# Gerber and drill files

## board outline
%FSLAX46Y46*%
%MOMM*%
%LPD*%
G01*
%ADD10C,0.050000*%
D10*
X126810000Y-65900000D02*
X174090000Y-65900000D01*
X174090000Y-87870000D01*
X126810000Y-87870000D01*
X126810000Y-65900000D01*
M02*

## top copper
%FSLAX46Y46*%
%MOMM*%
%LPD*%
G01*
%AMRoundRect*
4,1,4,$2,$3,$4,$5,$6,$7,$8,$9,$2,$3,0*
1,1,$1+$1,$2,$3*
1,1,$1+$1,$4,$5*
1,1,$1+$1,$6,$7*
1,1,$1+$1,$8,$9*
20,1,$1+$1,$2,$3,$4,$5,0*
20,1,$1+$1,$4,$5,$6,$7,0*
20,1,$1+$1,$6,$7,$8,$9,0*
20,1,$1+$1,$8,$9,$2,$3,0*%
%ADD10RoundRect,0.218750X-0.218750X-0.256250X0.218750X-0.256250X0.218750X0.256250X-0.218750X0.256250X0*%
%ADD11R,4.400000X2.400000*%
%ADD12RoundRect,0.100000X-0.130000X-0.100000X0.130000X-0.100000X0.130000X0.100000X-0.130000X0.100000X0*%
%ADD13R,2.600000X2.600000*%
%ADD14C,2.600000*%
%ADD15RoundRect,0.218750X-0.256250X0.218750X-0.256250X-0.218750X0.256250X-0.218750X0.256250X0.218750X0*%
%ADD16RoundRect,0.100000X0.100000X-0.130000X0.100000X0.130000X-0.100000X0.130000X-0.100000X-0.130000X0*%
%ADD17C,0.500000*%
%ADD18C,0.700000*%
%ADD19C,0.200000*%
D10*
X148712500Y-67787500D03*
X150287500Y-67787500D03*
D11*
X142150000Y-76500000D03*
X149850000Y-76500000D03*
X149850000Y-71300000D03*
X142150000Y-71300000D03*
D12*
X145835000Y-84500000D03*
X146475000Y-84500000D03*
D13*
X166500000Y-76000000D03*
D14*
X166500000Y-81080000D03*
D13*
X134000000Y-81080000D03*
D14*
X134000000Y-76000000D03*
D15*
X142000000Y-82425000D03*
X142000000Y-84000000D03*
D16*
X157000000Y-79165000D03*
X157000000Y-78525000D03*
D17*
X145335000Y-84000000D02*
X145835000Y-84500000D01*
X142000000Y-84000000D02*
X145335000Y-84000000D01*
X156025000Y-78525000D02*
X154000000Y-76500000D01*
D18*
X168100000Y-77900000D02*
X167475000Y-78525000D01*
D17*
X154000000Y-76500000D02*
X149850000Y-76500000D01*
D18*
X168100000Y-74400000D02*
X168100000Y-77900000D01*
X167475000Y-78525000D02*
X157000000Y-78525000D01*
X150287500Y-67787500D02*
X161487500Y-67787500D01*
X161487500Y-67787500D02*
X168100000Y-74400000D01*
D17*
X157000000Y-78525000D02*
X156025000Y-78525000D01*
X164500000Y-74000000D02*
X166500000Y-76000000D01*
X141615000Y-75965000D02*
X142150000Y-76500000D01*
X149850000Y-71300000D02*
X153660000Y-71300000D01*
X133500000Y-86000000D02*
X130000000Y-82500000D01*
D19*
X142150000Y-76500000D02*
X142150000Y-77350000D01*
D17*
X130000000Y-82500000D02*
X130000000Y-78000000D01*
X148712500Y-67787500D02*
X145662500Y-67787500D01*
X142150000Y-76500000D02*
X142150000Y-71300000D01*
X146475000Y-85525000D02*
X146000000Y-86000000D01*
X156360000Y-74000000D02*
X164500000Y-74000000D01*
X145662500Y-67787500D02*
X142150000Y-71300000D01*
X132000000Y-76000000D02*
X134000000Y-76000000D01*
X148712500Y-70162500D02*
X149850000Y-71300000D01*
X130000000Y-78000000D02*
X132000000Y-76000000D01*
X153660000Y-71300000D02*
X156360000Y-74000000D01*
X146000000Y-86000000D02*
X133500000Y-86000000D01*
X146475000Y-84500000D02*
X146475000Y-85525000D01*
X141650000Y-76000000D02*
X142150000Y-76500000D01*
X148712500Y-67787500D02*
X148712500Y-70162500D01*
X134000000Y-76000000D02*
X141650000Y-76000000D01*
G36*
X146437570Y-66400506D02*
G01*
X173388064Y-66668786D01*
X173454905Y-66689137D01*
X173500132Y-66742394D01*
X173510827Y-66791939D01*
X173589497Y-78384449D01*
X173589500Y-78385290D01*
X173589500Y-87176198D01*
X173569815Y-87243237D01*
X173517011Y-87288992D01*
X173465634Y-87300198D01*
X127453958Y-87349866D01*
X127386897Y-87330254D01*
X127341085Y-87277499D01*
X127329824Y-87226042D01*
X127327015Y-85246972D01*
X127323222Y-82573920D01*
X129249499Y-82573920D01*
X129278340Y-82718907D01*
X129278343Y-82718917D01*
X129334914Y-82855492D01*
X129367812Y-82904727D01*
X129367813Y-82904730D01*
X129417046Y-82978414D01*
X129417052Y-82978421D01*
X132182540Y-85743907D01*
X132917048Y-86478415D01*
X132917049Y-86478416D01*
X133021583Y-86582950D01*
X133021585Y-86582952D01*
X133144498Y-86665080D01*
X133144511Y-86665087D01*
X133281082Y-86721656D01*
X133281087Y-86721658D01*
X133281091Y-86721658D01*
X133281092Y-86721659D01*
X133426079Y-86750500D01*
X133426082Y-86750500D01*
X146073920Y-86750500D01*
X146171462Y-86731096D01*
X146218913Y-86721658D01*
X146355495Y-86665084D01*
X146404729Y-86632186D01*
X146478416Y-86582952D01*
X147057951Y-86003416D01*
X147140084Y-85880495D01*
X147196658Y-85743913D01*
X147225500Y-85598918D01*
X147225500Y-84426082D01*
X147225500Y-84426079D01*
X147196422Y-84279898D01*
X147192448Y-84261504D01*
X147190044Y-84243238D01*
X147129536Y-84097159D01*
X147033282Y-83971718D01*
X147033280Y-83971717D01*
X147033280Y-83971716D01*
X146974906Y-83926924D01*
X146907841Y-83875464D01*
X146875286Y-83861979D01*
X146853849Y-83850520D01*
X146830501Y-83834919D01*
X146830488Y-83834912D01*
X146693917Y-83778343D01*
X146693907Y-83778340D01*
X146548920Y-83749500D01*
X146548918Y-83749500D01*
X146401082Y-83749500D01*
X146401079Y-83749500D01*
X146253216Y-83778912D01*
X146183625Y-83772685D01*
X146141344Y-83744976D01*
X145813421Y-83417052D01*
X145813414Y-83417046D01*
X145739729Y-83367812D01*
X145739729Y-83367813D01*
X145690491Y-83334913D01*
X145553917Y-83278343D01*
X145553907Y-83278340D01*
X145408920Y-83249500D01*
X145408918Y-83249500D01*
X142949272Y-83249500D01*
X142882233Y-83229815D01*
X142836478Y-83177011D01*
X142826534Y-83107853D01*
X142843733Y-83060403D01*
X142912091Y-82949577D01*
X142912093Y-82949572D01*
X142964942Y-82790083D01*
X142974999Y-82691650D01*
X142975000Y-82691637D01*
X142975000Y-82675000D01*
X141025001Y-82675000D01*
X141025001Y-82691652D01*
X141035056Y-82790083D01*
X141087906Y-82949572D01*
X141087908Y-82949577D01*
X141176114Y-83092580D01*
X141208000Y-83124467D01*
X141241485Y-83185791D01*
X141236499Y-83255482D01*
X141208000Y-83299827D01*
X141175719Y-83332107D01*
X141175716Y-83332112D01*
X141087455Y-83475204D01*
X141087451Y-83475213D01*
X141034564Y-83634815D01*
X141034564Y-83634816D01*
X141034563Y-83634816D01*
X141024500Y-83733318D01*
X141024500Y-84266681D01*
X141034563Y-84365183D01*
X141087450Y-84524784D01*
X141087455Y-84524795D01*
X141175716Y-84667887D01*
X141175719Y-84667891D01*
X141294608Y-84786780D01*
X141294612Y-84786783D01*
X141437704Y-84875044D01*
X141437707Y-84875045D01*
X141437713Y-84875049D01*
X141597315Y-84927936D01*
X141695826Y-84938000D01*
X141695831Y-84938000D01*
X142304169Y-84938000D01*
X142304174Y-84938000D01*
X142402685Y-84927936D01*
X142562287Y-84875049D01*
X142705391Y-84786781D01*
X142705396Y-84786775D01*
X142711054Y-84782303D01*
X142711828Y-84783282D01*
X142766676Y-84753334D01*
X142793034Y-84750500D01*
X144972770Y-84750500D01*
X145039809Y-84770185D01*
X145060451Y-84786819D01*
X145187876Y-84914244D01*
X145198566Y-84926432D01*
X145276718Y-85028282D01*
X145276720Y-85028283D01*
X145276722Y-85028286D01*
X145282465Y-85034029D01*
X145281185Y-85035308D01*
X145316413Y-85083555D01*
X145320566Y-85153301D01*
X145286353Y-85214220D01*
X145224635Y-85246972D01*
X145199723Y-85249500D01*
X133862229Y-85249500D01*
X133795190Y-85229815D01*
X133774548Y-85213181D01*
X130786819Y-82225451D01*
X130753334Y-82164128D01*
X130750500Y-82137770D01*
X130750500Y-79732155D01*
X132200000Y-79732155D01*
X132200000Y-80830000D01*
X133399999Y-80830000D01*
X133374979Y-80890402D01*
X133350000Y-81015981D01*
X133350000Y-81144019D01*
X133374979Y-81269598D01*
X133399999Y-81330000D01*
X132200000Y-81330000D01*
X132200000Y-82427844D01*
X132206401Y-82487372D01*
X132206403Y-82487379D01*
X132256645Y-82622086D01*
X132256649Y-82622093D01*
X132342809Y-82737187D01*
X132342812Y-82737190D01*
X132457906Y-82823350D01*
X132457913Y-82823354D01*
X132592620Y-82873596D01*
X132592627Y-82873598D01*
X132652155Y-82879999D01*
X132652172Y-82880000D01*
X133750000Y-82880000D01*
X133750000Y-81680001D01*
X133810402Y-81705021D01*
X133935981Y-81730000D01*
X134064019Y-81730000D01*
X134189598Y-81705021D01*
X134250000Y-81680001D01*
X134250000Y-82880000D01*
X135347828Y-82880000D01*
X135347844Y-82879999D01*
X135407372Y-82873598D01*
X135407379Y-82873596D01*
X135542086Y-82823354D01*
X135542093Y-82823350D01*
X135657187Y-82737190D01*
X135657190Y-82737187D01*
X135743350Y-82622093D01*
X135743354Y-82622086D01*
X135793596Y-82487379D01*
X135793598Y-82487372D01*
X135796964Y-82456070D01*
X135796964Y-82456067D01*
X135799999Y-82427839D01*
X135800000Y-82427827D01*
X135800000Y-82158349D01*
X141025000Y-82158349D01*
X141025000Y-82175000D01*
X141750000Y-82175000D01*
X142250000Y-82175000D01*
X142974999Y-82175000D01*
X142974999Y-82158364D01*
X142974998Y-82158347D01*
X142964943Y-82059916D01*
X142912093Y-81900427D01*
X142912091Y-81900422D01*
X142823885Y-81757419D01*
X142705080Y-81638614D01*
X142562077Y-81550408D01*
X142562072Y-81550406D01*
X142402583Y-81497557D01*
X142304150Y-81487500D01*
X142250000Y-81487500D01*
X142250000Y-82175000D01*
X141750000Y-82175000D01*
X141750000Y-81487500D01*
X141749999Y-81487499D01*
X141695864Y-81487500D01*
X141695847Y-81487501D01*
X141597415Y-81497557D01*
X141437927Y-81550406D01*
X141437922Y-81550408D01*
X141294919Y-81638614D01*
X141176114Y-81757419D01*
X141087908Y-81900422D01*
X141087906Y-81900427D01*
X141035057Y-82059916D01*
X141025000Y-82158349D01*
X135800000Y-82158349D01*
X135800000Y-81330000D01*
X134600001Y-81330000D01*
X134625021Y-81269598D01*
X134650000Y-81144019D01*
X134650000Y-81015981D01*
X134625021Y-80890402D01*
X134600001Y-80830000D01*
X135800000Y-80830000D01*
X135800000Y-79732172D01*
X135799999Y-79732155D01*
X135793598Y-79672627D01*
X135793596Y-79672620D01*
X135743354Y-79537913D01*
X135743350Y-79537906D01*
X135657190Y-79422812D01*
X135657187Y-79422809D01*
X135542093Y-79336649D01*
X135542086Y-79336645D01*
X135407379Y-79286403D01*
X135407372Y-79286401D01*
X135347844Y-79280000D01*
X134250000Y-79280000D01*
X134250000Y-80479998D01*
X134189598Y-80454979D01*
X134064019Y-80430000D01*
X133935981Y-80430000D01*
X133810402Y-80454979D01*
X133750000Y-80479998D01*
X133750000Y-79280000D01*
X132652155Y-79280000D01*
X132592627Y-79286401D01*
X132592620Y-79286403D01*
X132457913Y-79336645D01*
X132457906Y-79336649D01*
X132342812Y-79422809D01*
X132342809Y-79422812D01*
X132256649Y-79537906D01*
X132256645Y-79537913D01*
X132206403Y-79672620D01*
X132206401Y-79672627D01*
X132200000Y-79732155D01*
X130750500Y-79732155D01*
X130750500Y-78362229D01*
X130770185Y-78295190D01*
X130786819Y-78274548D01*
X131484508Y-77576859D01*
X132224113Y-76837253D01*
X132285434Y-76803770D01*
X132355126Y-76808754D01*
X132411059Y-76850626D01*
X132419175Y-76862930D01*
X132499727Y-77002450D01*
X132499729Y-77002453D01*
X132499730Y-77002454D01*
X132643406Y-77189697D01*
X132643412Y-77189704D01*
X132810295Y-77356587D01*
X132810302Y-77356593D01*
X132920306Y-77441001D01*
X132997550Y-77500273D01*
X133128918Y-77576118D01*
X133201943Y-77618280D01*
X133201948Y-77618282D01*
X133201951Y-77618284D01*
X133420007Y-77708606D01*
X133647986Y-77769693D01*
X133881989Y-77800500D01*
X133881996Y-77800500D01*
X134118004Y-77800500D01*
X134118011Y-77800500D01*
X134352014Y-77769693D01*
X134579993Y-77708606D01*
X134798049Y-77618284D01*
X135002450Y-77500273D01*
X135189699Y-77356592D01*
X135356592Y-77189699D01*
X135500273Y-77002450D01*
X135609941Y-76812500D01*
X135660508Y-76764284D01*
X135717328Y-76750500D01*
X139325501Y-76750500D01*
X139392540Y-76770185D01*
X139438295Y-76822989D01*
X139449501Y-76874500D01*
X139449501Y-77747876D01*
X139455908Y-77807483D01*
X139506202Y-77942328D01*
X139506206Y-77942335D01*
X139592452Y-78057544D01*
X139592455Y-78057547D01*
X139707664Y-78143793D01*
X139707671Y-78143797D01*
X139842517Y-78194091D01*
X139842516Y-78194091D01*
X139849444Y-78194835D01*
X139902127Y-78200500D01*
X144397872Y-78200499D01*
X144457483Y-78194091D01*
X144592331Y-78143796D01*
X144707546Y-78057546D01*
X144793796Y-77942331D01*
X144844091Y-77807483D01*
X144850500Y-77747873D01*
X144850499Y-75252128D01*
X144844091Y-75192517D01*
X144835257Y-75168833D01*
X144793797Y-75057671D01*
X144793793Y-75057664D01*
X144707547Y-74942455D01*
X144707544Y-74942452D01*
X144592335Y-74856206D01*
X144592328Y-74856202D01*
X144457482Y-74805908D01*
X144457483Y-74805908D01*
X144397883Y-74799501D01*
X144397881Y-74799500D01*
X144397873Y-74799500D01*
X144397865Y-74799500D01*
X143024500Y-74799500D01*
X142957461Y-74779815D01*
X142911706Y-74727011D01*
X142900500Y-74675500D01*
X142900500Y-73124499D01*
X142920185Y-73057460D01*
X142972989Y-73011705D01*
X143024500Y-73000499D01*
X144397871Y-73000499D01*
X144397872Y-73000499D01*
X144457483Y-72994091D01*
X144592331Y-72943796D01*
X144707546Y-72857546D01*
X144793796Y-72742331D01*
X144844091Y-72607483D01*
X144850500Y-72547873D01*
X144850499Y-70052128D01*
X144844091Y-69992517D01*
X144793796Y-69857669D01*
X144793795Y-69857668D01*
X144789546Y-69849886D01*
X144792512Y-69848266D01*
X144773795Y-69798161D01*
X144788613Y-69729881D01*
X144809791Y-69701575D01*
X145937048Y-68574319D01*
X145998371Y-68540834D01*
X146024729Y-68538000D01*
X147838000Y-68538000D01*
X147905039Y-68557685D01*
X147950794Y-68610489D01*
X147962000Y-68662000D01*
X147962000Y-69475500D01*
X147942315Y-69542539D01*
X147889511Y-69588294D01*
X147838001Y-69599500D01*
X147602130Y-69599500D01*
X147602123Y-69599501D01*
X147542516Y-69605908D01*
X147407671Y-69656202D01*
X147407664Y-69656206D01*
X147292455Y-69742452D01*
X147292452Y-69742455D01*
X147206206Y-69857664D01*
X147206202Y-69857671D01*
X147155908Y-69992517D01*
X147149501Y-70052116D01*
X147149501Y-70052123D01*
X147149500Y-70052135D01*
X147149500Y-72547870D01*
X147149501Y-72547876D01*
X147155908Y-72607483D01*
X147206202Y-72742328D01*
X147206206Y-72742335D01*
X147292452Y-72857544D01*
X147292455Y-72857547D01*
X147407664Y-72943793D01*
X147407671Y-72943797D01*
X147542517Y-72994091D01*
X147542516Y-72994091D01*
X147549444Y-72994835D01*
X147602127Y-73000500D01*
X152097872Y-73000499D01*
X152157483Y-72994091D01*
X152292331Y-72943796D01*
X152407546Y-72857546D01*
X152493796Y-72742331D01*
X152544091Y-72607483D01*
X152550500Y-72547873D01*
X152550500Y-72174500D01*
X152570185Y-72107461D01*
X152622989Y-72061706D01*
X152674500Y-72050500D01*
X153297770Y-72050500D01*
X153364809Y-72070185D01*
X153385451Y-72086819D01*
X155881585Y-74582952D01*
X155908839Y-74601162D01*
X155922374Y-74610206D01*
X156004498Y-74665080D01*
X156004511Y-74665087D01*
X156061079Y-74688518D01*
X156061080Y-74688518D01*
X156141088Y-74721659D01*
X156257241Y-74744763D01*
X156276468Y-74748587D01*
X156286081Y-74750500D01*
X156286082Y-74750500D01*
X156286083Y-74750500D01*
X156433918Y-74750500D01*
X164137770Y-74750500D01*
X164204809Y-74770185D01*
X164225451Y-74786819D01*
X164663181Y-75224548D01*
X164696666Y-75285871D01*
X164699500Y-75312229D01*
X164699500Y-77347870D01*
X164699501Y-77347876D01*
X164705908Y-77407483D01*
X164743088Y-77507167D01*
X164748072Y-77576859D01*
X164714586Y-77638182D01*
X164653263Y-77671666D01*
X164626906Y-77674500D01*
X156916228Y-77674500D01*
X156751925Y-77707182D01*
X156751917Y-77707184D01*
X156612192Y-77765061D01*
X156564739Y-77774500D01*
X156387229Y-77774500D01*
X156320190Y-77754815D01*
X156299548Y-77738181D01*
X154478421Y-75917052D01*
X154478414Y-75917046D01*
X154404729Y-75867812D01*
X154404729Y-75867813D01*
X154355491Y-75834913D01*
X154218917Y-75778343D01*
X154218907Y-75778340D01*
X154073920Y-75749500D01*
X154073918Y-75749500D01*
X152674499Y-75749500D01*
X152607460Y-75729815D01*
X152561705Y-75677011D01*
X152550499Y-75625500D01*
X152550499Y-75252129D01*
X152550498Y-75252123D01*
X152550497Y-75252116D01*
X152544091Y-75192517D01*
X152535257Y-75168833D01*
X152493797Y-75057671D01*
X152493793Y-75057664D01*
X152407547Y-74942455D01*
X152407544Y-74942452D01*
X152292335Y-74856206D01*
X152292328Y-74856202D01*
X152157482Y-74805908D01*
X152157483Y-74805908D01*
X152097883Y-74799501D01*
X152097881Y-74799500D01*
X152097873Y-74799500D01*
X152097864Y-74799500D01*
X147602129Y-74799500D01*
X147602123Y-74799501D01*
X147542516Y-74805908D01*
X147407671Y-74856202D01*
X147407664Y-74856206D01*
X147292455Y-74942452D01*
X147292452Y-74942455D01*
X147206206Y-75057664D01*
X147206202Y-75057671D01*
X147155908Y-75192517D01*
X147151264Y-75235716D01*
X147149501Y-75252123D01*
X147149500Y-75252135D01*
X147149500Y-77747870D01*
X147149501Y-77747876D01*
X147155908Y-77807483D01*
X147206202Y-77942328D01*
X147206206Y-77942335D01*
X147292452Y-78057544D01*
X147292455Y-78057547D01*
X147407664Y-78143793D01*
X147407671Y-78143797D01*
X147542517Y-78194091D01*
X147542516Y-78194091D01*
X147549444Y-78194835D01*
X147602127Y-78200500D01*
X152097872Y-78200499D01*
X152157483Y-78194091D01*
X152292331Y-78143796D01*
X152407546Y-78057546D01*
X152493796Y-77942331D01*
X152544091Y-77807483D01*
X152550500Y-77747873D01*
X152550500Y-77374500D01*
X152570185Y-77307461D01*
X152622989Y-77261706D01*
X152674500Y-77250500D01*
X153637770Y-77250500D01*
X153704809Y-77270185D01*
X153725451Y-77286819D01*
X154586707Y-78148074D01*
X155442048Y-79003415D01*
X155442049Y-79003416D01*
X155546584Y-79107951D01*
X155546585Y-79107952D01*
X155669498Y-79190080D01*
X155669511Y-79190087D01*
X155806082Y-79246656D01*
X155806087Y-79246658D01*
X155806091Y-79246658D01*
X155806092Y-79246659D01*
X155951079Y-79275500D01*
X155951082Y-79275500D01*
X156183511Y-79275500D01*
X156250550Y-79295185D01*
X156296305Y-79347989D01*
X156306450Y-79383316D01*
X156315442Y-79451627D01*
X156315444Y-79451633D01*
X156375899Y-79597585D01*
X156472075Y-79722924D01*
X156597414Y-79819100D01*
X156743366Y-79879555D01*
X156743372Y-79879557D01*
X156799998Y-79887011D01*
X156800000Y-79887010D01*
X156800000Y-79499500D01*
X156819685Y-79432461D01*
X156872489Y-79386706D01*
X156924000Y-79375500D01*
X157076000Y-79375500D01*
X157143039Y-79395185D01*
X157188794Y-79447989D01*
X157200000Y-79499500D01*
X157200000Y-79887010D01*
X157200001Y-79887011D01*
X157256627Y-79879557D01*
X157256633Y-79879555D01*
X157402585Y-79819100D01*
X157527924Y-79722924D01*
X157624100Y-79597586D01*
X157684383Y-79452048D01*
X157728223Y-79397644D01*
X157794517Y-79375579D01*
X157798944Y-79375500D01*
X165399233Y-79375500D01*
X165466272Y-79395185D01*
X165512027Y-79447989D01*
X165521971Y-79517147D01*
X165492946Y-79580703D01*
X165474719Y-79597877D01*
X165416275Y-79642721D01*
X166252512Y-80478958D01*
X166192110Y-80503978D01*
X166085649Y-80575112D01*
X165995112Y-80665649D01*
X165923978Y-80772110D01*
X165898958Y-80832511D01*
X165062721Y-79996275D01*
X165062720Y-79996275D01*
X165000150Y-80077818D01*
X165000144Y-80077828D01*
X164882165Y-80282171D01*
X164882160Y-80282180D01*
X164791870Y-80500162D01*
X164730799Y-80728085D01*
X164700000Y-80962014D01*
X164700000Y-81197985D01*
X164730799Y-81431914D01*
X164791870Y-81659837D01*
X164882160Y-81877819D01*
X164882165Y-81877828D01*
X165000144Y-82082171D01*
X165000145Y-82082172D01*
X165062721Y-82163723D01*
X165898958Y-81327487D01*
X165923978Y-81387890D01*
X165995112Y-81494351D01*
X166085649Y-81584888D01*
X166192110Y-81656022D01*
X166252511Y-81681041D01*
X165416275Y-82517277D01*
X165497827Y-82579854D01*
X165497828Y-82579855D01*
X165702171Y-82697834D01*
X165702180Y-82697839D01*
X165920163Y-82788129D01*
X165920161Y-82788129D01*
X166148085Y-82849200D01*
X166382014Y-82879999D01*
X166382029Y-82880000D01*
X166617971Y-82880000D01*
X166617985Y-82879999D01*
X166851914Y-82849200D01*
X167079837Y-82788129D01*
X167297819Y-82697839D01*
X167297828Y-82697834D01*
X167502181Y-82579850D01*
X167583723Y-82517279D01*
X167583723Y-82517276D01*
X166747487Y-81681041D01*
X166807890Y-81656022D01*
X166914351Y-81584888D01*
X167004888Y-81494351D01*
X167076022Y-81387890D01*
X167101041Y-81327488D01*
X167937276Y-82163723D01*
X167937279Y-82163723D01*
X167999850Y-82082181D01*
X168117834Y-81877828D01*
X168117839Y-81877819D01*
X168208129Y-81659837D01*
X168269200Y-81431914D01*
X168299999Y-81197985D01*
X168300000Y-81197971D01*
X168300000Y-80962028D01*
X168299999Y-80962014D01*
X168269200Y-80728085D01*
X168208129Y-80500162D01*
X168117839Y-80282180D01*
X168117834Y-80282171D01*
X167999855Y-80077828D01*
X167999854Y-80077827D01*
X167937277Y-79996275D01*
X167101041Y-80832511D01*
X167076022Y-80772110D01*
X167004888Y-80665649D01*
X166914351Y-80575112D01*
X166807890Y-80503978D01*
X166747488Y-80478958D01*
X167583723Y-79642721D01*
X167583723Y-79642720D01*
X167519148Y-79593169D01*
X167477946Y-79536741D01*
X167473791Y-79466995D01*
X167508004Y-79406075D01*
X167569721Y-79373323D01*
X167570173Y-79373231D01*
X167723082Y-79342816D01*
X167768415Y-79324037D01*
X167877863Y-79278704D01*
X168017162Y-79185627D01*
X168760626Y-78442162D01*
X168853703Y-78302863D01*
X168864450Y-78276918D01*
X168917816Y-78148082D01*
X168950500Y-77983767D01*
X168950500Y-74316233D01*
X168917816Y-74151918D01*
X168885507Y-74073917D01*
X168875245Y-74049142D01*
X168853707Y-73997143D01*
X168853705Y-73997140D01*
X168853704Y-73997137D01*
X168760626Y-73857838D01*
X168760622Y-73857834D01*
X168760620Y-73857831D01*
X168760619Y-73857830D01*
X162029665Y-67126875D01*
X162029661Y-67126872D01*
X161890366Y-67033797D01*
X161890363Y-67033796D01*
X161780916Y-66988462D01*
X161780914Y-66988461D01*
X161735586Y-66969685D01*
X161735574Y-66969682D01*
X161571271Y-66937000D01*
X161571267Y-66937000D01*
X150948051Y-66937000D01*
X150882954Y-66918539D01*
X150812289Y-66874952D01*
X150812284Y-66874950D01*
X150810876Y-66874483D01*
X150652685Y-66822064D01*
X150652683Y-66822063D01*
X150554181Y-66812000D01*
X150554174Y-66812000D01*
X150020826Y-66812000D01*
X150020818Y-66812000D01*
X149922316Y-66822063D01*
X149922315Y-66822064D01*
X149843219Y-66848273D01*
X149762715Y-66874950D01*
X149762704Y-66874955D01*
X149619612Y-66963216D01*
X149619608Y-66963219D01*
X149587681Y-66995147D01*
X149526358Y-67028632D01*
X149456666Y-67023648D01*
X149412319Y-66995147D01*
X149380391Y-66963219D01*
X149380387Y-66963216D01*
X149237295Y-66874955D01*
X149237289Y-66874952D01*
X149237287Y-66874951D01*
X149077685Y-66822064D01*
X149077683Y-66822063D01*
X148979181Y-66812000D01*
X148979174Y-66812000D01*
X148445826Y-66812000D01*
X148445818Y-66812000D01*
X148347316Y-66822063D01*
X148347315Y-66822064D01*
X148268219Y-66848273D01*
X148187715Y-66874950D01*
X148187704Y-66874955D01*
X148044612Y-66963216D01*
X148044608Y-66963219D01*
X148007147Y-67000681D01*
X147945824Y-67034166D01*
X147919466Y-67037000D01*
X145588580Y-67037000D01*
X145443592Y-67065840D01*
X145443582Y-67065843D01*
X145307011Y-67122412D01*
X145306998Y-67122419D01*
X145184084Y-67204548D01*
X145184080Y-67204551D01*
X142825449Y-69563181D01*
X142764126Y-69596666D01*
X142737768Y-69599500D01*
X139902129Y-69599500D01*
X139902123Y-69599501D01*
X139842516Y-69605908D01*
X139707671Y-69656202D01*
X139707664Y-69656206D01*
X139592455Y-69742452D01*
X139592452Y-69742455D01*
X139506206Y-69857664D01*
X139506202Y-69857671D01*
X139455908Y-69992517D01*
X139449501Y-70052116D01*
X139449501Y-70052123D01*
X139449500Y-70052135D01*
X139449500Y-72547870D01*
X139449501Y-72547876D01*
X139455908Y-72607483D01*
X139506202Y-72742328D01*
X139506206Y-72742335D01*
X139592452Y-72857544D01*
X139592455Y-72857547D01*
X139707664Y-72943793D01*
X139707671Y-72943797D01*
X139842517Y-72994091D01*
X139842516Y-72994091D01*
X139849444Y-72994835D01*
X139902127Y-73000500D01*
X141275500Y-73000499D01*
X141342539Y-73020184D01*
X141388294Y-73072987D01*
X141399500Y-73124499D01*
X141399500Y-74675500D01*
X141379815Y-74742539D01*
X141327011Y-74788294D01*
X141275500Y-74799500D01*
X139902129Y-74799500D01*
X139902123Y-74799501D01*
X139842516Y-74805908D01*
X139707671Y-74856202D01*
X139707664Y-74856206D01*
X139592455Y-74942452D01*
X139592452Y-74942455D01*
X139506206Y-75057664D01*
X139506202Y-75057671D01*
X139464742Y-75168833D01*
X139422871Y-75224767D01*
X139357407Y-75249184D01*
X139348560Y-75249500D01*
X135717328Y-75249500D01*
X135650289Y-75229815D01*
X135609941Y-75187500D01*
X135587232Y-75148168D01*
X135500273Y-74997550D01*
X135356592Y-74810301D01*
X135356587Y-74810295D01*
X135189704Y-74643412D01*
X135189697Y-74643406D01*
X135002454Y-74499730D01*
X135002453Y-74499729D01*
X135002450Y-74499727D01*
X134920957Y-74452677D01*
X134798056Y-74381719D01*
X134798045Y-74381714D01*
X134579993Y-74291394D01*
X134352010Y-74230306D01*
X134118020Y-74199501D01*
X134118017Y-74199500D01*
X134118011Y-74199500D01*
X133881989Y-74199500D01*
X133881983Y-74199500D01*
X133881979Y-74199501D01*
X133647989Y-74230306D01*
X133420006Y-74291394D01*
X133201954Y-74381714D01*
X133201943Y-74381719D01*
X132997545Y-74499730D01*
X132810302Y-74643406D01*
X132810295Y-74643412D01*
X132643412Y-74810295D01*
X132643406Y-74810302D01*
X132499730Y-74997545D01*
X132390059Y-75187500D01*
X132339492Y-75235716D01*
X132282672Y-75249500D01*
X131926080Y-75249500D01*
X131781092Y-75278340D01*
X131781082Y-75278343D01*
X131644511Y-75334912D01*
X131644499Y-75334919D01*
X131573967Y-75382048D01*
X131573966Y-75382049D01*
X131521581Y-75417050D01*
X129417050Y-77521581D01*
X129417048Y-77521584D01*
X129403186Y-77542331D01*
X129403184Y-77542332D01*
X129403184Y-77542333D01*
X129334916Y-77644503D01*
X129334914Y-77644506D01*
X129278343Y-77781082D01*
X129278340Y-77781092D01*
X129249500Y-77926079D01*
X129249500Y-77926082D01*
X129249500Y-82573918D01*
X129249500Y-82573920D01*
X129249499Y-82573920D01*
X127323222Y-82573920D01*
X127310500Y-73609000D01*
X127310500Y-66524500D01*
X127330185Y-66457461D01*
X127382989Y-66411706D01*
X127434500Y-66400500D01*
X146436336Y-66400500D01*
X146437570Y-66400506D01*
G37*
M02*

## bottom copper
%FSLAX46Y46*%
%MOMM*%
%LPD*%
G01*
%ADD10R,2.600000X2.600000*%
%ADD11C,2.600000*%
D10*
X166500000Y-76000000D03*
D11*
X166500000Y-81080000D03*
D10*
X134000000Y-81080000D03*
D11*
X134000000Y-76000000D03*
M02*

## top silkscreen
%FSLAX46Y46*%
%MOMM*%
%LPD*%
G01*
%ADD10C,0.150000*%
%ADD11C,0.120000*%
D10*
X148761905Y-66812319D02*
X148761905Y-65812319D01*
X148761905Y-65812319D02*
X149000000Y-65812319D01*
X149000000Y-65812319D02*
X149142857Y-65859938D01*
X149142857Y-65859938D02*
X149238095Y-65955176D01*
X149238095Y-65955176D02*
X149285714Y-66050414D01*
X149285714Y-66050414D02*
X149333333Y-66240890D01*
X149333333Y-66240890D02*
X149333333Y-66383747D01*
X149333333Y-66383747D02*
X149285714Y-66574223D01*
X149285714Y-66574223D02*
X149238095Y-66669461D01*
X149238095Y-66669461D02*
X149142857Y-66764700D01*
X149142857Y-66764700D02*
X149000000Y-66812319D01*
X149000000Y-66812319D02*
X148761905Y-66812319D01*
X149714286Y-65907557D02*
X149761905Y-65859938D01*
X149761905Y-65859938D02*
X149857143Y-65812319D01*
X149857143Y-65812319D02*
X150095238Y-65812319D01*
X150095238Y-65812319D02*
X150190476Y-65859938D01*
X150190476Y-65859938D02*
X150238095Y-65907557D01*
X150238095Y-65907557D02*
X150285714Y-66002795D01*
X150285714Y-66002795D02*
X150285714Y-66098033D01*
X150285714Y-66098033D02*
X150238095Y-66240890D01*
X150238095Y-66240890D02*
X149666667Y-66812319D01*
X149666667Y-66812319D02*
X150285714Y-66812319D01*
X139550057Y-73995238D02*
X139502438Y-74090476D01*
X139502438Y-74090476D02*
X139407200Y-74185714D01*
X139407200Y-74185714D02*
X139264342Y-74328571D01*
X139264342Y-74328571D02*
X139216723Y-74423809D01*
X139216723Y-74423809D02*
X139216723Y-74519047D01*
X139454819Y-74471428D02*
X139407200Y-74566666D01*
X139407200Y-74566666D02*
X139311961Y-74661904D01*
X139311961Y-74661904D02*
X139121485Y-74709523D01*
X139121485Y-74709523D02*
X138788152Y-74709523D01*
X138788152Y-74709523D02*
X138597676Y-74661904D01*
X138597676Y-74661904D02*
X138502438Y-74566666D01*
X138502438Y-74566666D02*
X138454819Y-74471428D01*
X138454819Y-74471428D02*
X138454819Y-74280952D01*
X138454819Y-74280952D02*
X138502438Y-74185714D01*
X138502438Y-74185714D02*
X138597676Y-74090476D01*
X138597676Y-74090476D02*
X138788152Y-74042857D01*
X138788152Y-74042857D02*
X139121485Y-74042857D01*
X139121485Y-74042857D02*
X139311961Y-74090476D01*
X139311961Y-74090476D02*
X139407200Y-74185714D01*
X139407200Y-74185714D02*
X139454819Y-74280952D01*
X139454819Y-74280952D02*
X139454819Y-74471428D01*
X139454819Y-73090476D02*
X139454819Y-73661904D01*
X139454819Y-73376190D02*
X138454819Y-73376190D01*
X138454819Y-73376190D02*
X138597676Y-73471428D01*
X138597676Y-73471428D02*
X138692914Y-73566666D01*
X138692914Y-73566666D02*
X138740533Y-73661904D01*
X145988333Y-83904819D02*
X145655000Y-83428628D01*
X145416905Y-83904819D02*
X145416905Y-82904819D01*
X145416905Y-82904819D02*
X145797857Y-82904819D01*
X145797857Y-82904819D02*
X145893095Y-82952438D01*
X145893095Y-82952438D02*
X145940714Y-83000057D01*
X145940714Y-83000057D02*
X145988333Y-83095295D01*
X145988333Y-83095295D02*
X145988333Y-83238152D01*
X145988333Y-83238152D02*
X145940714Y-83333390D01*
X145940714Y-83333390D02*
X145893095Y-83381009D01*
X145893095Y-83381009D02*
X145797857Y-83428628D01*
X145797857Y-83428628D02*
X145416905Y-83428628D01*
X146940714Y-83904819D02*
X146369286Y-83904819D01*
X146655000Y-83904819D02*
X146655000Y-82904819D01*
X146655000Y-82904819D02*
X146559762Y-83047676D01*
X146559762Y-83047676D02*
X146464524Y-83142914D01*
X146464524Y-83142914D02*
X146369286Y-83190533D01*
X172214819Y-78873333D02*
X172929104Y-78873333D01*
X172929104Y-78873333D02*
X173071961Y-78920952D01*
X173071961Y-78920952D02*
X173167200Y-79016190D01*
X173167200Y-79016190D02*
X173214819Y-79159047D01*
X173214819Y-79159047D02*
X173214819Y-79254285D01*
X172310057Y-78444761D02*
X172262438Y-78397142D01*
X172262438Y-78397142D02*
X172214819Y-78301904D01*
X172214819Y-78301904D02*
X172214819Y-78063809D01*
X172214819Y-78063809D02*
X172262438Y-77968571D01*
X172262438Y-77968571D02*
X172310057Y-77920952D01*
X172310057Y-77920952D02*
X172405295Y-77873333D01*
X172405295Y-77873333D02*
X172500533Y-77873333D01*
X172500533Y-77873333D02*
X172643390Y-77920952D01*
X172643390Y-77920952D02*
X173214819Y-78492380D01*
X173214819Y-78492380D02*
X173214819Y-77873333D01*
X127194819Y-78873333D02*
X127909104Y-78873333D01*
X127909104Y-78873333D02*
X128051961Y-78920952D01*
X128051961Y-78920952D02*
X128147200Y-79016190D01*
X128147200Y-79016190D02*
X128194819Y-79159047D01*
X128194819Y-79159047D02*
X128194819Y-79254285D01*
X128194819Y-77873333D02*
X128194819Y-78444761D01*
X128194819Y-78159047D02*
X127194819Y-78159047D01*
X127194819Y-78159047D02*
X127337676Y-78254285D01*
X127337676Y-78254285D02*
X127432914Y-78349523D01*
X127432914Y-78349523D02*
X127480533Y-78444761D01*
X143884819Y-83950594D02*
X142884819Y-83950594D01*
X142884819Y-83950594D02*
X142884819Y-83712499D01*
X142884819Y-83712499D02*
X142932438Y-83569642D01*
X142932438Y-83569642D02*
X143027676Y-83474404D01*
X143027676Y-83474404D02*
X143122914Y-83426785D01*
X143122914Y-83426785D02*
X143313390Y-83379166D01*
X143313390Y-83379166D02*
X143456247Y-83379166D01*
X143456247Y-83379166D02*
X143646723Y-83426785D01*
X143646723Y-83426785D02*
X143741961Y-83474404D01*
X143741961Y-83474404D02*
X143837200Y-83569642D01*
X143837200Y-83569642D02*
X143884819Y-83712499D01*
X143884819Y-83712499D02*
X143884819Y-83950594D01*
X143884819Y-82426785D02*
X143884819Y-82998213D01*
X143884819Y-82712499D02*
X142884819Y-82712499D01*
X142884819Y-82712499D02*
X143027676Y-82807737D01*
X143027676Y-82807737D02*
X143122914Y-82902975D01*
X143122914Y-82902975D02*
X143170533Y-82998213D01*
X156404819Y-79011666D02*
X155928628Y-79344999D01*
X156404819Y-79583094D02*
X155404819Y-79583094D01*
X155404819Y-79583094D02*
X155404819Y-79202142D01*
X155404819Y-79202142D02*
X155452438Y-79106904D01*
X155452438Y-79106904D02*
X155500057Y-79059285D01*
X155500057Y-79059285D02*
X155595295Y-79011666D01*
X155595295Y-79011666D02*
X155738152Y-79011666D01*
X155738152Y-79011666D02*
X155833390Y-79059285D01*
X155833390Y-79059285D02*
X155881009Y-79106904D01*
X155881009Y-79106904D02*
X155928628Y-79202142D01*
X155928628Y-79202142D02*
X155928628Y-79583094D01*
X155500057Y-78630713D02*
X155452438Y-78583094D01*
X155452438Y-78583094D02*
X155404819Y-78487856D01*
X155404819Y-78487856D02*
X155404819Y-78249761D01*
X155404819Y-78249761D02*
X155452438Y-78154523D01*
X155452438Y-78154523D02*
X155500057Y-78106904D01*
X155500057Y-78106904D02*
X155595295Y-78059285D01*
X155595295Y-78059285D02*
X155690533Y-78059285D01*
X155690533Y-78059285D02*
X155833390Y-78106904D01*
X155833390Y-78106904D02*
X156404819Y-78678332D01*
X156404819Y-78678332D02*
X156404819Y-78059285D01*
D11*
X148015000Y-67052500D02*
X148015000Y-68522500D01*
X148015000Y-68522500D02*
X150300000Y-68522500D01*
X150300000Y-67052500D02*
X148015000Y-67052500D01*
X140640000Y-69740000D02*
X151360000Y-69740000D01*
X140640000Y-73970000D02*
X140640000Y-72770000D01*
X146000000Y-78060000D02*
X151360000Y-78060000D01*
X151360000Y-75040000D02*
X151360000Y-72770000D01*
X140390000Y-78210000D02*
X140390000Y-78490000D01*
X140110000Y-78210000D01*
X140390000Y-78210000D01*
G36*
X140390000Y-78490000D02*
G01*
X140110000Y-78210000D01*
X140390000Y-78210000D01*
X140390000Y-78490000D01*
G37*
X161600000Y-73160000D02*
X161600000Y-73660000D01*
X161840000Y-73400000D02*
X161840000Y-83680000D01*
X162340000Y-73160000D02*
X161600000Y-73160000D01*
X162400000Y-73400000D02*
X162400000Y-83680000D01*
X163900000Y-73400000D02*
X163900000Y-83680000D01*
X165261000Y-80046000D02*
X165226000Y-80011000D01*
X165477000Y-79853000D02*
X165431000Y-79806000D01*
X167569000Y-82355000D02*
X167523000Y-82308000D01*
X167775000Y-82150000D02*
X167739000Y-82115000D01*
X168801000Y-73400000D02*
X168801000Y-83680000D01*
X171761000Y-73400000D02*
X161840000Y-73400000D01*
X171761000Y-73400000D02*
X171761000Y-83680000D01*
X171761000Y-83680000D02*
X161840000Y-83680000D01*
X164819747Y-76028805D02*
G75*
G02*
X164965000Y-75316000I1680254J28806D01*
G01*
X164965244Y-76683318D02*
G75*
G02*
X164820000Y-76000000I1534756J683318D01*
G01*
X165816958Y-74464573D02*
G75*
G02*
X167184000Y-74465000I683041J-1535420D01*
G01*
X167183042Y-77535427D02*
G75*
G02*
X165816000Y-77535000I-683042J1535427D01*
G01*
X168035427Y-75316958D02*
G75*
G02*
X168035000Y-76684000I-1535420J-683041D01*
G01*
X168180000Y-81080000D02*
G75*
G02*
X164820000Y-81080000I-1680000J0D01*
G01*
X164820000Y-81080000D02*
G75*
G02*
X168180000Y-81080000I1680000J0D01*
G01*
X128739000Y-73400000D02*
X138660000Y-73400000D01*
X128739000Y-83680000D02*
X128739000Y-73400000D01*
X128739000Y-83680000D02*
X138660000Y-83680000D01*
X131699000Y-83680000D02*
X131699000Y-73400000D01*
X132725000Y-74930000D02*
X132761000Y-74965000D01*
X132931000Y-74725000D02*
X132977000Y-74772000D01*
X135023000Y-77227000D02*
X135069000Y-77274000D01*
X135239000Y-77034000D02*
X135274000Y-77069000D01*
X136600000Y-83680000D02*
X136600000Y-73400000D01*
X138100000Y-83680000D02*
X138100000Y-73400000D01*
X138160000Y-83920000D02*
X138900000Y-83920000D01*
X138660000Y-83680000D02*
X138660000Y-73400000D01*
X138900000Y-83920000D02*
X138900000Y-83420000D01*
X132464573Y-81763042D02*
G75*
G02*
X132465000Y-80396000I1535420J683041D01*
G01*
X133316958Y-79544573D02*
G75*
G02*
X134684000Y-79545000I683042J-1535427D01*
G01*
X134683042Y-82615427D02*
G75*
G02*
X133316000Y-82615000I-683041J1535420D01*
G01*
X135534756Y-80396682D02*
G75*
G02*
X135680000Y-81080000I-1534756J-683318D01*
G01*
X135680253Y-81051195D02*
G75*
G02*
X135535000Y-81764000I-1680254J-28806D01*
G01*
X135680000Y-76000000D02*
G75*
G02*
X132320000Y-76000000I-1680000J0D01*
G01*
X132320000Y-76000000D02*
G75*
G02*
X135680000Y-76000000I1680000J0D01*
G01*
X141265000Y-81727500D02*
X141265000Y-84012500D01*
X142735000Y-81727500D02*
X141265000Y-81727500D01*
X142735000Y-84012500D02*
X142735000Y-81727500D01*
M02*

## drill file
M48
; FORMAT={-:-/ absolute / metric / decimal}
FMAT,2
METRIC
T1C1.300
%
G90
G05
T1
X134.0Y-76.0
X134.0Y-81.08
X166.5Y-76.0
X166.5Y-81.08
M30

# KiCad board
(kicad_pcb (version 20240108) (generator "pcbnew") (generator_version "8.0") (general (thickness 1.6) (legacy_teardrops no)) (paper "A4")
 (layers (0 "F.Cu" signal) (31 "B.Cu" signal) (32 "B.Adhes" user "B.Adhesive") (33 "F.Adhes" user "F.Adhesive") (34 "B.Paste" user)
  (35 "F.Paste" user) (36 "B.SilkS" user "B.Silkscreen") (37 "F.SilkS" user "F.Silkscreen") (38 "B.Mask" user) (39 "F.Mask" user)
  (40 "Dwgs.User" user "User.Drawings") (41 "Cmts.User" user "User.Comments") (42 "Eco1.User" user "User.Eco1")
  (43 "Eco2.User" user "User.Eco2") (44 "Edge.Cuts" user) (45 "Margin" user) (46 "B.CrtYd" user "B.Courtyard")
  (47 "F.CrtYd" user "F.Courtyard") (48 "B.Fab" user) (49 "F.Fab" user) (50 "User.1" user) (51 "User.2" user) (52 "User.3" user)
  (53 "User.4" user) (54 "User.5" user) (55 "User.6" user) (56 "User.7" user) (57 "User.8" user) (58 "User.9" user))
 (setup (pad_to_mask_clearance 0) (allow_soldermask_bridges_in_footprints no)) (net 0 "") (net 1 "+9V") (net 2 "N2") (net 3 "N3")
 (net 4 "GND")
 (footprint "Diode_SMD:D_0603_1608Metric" (layer "F.Cu") (at 149.5 67.7875)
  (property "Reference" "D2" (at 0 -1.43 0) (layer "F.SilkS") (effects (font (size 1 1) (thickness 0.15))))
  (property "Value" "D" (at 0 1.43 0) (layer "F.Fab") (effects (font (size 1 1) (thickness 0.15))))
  (fp_line (start -1.485 -0.735) (end -1.485 0.735) (stroke (width 0.12) (type solid)) (layer "F.SilkS"))
  (fp_line (start -1.485 0.735) (end 0.8 0.735) (stroke (width 0.12) (type solid)) (layer "F.SilkS"))
  (fp_line (start 0.8 -0.735) (end -1.485 -0.735) (stroke (width 0.12) (type solid)) (layer "F.SilkS"))
  (pad "1" smd roundrect (at -0.7875 0) (size 0.875 0.95) (layers "F.Cu" "F.Paste" "F.Mask") (roundrect_rratio 0.25) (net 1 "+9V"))
  (pad "2" smd roundrect (at 0.7875 0) (size 0.875 0.95) (layers "F.Cu" "F.Paste" "F.Mask") (roundrect_rratio 0.25) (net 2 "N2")))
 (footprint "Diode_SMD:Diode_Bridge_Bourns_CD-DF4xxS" (layer "F.Cu") (at 146 73.9 90)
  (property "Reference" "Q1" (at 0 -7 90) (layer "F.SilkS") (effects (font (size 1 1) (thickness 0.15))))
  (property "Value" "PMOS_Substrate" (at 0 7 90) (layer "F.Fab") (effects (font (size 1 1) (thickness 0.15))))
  (fp_line (start 4.16 -5.36) (end 4.16 5.36) (stroke (width 0.12) (type solid)) (layer "F.SilkS"))
  (fp_line (start -0.07 -5.36) (end 1.13 -5.36) (stroke (width 0.12) (type solid)) (layer "F.SilkS"))
  (fp_line (start -4.16 0) (end -4.16 5.36) (stroke (width 0.12) (type solid)) (layer "F.SilkS"))
  (fp_line (start -1.14 5.36) (end 1.13 5.36) (stroke (width 0.12) (type solid)) (layer "F.SilkS"))
  (fp_poly
   (pts (xy -4.31 -5.61) (xy -4.59 -5.61) (xy -4.31 -5.89) (xy -4.31 -5.61)) (stroke (width 0.12) (type solid)) (fill solid)
   (layer "F.SilkS"))
  (pad "1" smd rect (at -2.6 -3.85 90) (size 2.4 4.4) (layers "F.Cu" "F.Paste" "F.Mask") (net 1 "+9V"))
  (pad "2" smd rect (at -2.6 3.85 90) (size 2.4 4.4) (layers "F.Cu" "F.Paste" "F.Mask") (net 2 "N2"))
  (pad "3" smd rect (at 2.6 3.85 90) (size 2.4 4.4) (layers "F.Cu" "F.Paste" "F.Mask") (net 1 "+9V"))
  (pad "4" smd rect (at 2.6 -3.85 90) (size 2.4 4.4) (layers "F.Cu" "F.Paste" "F.Mask") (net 1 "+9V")))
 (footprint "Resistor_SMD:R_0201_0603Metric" (layer "F.Cu") (at 146.155 84.5)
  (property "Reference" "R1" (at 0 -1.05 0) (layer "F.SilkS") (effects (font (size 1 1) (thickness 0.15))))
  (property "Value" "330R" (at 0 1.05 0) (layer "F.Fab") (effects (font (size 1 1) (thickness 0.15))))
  (pad "" smd roundrect (at -0.345 0) (size 0.318 0.36) (layers "F.Paste") (roundrect_rratio 0.25))
  (pad "" smd roundrect (at 0.345 0) (size 0.318 0.36) (layers "F.Paste") (roundrect_rratio 0.25))
  (pad "1" smd roundrect (at -0.32 0) (size 0.46 0.4) (layers "F.Cu" "F.Mask") (roundrect_rratio 0.25) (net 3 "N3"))
  (pad "2" smd roundrect (at 0.32 0) (size 0.46 0.4) (layers "F.Cu" "F.Mask") (roundrect_rratio 0.25) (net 1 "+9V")))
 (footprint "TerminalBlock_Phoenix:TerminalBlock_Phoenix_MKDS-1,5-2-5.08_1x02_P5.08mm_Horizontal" (layer "F.Cu") (at 166.5 76 -90)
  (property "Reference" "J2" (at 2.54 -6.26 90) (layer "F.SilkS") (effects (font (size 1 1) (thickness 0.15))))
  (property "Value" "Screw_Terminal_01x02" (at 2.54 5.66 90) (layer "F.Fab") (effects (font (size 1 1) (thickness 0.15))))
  (fp_line (start -2.84 4.9) (end -2.34 4.9) (stroke (width 0.12) (type solid)) (layer "F.SilkS"))
  (fp_line (start -2.6 4.66) (end 7.68 4.66) (stroke (width 0.12) (type solid)) (layer "F.SilkS"))
  (fp_line (start -2.84 4.16) (end -2.84 4.9) (stroke (width 0.12) (type solid)) (layer "F.SilkS"))
  (fp_line (start -2.6 4.1) (end 7.68 4.1) (stroke (width 0.12) (type solid)) (layer "F.SilkS"))
  (fp_line (start -2.6 2.6) (end 7.68 2.6) (stroke (width 0.12) (type solid)) (layer "F.SilkS"))
  (fp_line (start 4.046 1.239) (end 4.011 1.274) (stroke (width 0.12) (type solid)) (layer "F.SilkS"))
  (fp_line (start 3.853 1.023) (end 3.806 1.069) (stroke (width 0.12) (type solid)) (layer "F.SilkS"))
  (fp_line (start 6.355 -1.069) (end 6.308 -1.023) (stroke (width 0.12) (type solid)) (layer "F.SilkS"))
  (fp_line (start 6.15 -1.275) (end 6.115 -1.239) (stroke (width 0.12) (type solid)) (layer "F.SilkS"))
  (fp_line (start -2.6 -2.301) (end 7.68 -2.301) (stroke (width 0.12) (type solid)) (layer "F.SilkS"))
  (fp_line (start -2.6 -5.261) (end -2.6 4.66) (stroke (width 0.12) (type solid)) (layer "F.SilkS"))
  (fp_line (start -2.6 -5.261) (end 7.68 -5.261) (stroke (width 0.12) (type solid)) (layer "F.SilkS"))
  (fp_line (start 7.68 -5.261) (end 7.68 4.66) (stroke (width 0.12) (type solid)) (layer "F.SilkS"))
  (fp_arc (start 0.028805 1.680253) (mid -0.335551 1.646659) (end -0.684 1.535) (stroke (width 0.12) (type solid)) (layer "F.SilkS"))
  (fp_arc (start 0.683318 1.534756) (mid 0.349292 1.643288) (end 0 1.68) (stroke (width 0.12) (type solid)) (layer "F.SilkS"))
  (fp_arc (start -1.535427 0.683042) (mid -1.680501 -0.000524) (end -1.535 -0.684) (stroke (width 0.12) (type solid)) (layer "F.SilkS"))
  (fp_arc (start 1.535427 -0.683042) (mid 1.680501 0.000524) (end 1.535 0.684) (stroke (width 0.12) (type solid)) (layer "F.SilkS"))
  (fp_arc (start -0.683042 -1.535427) (mid 0.000524 -1.680501) (end 0.684 -1.535) (stroke (width 0.12) (type solid)) (layer "F.SilkS"))
  (fp_circle (center 5.08 0) (end 6.76 0) (stroke (width 0.12) (type solid)) (fill none) (layer "F.SilkS"))
  (pad "1" thru_hole rect (at 0 0 270) (size 2.6 2.6) (drill 1.3) (layers "*.Cu" "*.Mask") (remove_unused_layers no) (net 1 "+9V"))
  (pad "2" thru_hole circle (at 5.08 0 270) (size 2.6 2.6) (drill 1.3) (layers "*.Cu" "*.Mask") (remove_unused_layers no) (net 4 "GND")))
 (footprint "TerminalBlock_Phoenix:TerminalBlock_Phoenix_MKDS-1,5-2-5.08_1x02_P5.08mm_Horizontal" (layer "F.Cu") (at 134 81.08 90)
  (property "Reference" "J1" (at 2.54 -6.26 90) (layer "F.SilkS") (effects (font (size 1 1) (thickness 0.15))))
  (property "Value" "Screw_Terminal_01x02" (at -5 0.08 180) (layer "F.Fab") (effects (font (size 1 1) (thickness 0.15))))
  (fp_line (start 7.68 -5.261) (end 7.68 4.66) (stroke (width 0.12) (type solid)) (layer "F.SilkS"))
  (fp_line (start -2.6 -5.261) (end 7.68 -5.261) (stroke (width 0.12) (type solid)) (layer "F.SilkS"))
  (fp_line (start -2.6 -5.261) (end -2.6 4.66) (stroke (width 0.12) (type solid)) (layer "F.SilkS"))
  (fp_line (start -2.6 -2.301) (end 7.68 -2.301) (stroke (width 0.12) (type solid)) (layer "F.SilkS"))
  (fp_line (start 6.15 -1.275) (end 6.115 -1.239) (stroke (width 0.12) (type solid)) (layer "F.SilkS"))
  (fp_line (start 6.355 -1.069) (end 6.308 -1.023) (stroke (width 0.12) (type solid)) (layer "F.SilkS"))
  (fp_line (start 3.853 1.023) (end 3.806 1.069) (stroke (width 0.12) (type solid)) (layer "F.SilkS"))
  (fp_line (start 4.046 1.239) (end 4.011 1.274) (stroke (width 0.12) (type solid)) (layer "F.SilkS"))
  (fp_line (start -2.6 2.6) (end 7.68 2.6) (stroke (width 0.12) (type solid)) (layer "F.SilkS"))
  (fp_line (start -2.6 4.1) (end 7.68 4.1) (stroke (width 0.12) (type solid)) (layer "F.SilkS"))
  (fp_line (start -2.84 4.16) (end -2.84 4.9) (stroke (width 0.12) (type solid)) (layer "F.SilkS"))
  (fp_line (start -2.6 4.66) (end 7.68 4.66) (stroke (width 0.12) (type solid)) (layer "F.SilkS"))
  (fp_line (start -2.84 4.9) (end -2.34 4.9) (stroke (width 0.12) (type solid)) (layer "F.SilkS"))
  (fp_arc (start -0.683042 -1.535427) (mid 0.000524 -1.680501) (end 0.684 -1.535) (stroke (width 0.12) (type solid)) (layer "F.SilkS"))
  (fp_arc (start 1.535427 -0.683042) (mid 1.680501 0.000524) (end 1.535 0.684) (stroke (width 0.12) (type solid)) (layer "F.SilkS"))
  (fp_arc (start -1.535427 0.683042) (mid -1.680501 -0.000524) (end -1.535 -0.684) (stroke (width 0.12) (type solid)) (layer "F.SilkS"))
  (fp_arc (start 0.683318 1.534756) (mid 0.349292 1.643288) (end 0 1.68) (stroke (width 0.12) (type solid)) (layer "F.SilkS"))
  (fp_arc (start 0.028805 1.680253) (mid -0.335551 1.646659) (end -0.684 1.535) (stroke (width 0.12) (type solid)) (layer "F.SilkS"))
  (fp_circle (center 5.08 0) (end 6.76 0) (stroke (width 0.12) (type solid)) (fill none) (layer "F.SilkS"))
  (pad "1" thru_hole rect (at 0 0 90) (size 2.6 2.6) (drill 1.3) (layers "*.Cu" "*.Mask") (remove_unused_layers no) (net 4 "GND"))
  (pad "2" thru_hole circle (at 5.08 0 90) (size 2.6 2.6) (drill 1.3) (layers "*.Cu" "*.Mask") (remove_unused_layers no) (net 1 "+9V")))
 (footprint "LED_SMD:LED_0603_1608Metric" (layer "F.Cu") (at 142 83.2125 -90)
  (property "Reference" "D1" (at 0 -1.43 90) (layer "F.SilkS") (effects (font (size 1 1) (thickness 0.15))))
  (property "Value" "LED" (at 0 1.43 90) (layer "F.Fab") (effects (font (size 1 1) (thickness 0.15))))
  (fp_line (start -1.485 0.735) (end 0.8 0.735) (stroke (width 0.12) (type solid)) (layer "F.SilkS"))
  (fp_line (start -1.485 -0.735) (end -1.485 0.735) (stroke (width 0.12) (type solid)) (layer "F.SilkS"))
  (fp_line (start 0.8 -0.735) (end -1.485 -0.735) (stroke (width 0.12) (type solid)) (layer "F.SilkS"))
  (pad "1" smd roundrect (at -0.7875 0 270) (size 0.875 0.95) (layers "F.Cu" "F.Paste" "F.Mask") (roundrect_rratio 0.25) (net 4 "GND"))
  (pad "2" smd roundrect (at 0.7875 0 270) (size 0.875 0.95) (layers "F.Cu" "F.Paste" "F.Mask") (roundrect_rratio 0.25) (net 3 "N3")))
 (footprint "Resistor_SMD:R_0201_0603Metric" (layer "F.Cu") (at 157 78.845 90)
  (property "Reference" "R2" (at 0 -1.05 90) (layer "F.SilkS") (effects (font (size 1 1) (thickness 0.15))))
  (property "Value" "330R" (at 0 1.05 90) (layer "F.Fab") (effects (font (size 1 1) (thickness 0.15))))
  (pad "" smd roundrect (at -0.345 0 90) (size 0.318 0.36) (layers "F.Paste") (roundrect_rratio 0.25))
  (pad "" smd roundrect (at 0.345 0 90) (size 0.318 0.36) (layers "F.Paste") (roundrect_rratio 0.25))
  (pad "1" smd roundrect (at -0.32 0 90) (size 0.46 0.4) (layers "F.Cu" "F.Mask") (roundrect_rratio 0.25) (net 4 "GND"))
  (pad "2" smd roundrect (at 0.32 0 90) (size 0.46 0.4) (layers "F.Cu" "F.Mask") (roundrect_rratio 0.25) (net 2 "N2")))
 (gr_rect (start 126.81 65.9) (end 174.09 87.87) (stroke (width 0.05) (type default)) (fill none) (layer "Edge.Cuts"))
 (segment (start 145.335 84) (end 145.835 84.5) (width 0.5) (layer "F.Cu") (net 3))
 (segment (start 142 84) (end 145.335 84) (width 0.5) (layer "F.Cu") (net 3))
 (segment (start 156.025 78.525) (end 154 76.5) (width 0.5) (layer "F.Cu") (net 2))
 (segment (start 168.1 77.9) (end 167.475 78.525) (width 0.7) (layer "F.Cu") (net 2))
 (segment (start 154 76.5) (end 149.85 76.5) (width 0.5) (layer "F.Cu") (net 2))
 (segment (start 168.1 74.4) (end 168.1 77.9) (width 0.7) (layer "F.Cu") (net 2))
 (segment (start 167.475 78.525) (end 157 78.525) (width 0.7) (layer "F.Cu") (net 2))
 (segment (start 150.2875 67.7875) (end 161.4875 67.7875) (width 0.7) (layer "F.Cu") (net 2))
 (segment (start 161.4875 67.7875) (end 168.1 74.4) (width 0.7) (layer "F.Cu") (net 2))
 (segment (start 157 78.525) (end 156.025 78.525) (width 0.5) (layer "F.Cu") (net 2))
 (segment (start 164.5 74) (end 166.5 76) (width 0.5) (layer "F.Cu") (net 1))
 (segment (start 141.615 75.965) (end 142.15 76.5) (width 0.5) (layer "F.Cu") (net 1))
 (segment (start 149.85 71.3) (end 153.66 71.3) (width 0.5) (layer "F.Cu") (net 1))
 (segment (start 133.5 86) (end 130 82.5) (width 0.5) (layer "F.Cu") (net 1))
 (segment (start 142.15 76.5) (end 142.15 77.35) (width 0.2) (layer "F.Cu") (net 1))
 (segment (start 130 82.5) (end 130 78) (width 0.5) (layer "F.Cu") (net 1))
 (segment (start 148.7125 67.7875) (end 145.6625 67.7875) (width 0.5) (layer "F.Cu") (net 1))
 (segment (start 142.15 76.5) (end 142.15 71.3) (width 0.5) (layer "F.Cu") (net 1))
 (segment (start 146.475 85.525) (end 146 86) (width 0.5) (layer "F.Cu") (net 1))
 (segment (start 156.36 74) (end 164.5 74) (width 0.5) (layer "F.Cu") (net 1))
 (segment (start 145.6625 67.7875) (end 142.15 71.3) (width 0.5) (layer "F.Cu") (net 1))
 (segment (start 132 76) (end 134 76) (width 0.5) (layer "F.Cu") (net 1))
 (segment (start 148.7125 70.1625) (end 149.85 71.3) (width 0.5) (layer "F.Cu") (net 1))
 (segment (start 130 78) (end 132 76) (width 0.5) (layer "F.Cu") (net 1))
 (segment (start 153.66 71.3) (end 156.36 74) (width 0.5) (layer "F.Cu") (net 1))
 (segment (start 146 86) (end 133.5 86) (width 0.5) (layer "F.Cu") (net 1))
 (segment (start 146.475 84.5) (end 146.475 85.525) (width 0.5) (layer "F.Cu") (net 1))
 (segment (start 141.65 76) (end 142.15 76.5) (width 0.5) (layer "F.Cu") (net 1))
 (segment (start 148.7125 67.7875) (end 148.7125 70.1625) (width 0.5) (layer "F.Cu") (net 1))
 (segment (start 134 76) (end 141.65 76) (width 0.5) (layer "F.Cu") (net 1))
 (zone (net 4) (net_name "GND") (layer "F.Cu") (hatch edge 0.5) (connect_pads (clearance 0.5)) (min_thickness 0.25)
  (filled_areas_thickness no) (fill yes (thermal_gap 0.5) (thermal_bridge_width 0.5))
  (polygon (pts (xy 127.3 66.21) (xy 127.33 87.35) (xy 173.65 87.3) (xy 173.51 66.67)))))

